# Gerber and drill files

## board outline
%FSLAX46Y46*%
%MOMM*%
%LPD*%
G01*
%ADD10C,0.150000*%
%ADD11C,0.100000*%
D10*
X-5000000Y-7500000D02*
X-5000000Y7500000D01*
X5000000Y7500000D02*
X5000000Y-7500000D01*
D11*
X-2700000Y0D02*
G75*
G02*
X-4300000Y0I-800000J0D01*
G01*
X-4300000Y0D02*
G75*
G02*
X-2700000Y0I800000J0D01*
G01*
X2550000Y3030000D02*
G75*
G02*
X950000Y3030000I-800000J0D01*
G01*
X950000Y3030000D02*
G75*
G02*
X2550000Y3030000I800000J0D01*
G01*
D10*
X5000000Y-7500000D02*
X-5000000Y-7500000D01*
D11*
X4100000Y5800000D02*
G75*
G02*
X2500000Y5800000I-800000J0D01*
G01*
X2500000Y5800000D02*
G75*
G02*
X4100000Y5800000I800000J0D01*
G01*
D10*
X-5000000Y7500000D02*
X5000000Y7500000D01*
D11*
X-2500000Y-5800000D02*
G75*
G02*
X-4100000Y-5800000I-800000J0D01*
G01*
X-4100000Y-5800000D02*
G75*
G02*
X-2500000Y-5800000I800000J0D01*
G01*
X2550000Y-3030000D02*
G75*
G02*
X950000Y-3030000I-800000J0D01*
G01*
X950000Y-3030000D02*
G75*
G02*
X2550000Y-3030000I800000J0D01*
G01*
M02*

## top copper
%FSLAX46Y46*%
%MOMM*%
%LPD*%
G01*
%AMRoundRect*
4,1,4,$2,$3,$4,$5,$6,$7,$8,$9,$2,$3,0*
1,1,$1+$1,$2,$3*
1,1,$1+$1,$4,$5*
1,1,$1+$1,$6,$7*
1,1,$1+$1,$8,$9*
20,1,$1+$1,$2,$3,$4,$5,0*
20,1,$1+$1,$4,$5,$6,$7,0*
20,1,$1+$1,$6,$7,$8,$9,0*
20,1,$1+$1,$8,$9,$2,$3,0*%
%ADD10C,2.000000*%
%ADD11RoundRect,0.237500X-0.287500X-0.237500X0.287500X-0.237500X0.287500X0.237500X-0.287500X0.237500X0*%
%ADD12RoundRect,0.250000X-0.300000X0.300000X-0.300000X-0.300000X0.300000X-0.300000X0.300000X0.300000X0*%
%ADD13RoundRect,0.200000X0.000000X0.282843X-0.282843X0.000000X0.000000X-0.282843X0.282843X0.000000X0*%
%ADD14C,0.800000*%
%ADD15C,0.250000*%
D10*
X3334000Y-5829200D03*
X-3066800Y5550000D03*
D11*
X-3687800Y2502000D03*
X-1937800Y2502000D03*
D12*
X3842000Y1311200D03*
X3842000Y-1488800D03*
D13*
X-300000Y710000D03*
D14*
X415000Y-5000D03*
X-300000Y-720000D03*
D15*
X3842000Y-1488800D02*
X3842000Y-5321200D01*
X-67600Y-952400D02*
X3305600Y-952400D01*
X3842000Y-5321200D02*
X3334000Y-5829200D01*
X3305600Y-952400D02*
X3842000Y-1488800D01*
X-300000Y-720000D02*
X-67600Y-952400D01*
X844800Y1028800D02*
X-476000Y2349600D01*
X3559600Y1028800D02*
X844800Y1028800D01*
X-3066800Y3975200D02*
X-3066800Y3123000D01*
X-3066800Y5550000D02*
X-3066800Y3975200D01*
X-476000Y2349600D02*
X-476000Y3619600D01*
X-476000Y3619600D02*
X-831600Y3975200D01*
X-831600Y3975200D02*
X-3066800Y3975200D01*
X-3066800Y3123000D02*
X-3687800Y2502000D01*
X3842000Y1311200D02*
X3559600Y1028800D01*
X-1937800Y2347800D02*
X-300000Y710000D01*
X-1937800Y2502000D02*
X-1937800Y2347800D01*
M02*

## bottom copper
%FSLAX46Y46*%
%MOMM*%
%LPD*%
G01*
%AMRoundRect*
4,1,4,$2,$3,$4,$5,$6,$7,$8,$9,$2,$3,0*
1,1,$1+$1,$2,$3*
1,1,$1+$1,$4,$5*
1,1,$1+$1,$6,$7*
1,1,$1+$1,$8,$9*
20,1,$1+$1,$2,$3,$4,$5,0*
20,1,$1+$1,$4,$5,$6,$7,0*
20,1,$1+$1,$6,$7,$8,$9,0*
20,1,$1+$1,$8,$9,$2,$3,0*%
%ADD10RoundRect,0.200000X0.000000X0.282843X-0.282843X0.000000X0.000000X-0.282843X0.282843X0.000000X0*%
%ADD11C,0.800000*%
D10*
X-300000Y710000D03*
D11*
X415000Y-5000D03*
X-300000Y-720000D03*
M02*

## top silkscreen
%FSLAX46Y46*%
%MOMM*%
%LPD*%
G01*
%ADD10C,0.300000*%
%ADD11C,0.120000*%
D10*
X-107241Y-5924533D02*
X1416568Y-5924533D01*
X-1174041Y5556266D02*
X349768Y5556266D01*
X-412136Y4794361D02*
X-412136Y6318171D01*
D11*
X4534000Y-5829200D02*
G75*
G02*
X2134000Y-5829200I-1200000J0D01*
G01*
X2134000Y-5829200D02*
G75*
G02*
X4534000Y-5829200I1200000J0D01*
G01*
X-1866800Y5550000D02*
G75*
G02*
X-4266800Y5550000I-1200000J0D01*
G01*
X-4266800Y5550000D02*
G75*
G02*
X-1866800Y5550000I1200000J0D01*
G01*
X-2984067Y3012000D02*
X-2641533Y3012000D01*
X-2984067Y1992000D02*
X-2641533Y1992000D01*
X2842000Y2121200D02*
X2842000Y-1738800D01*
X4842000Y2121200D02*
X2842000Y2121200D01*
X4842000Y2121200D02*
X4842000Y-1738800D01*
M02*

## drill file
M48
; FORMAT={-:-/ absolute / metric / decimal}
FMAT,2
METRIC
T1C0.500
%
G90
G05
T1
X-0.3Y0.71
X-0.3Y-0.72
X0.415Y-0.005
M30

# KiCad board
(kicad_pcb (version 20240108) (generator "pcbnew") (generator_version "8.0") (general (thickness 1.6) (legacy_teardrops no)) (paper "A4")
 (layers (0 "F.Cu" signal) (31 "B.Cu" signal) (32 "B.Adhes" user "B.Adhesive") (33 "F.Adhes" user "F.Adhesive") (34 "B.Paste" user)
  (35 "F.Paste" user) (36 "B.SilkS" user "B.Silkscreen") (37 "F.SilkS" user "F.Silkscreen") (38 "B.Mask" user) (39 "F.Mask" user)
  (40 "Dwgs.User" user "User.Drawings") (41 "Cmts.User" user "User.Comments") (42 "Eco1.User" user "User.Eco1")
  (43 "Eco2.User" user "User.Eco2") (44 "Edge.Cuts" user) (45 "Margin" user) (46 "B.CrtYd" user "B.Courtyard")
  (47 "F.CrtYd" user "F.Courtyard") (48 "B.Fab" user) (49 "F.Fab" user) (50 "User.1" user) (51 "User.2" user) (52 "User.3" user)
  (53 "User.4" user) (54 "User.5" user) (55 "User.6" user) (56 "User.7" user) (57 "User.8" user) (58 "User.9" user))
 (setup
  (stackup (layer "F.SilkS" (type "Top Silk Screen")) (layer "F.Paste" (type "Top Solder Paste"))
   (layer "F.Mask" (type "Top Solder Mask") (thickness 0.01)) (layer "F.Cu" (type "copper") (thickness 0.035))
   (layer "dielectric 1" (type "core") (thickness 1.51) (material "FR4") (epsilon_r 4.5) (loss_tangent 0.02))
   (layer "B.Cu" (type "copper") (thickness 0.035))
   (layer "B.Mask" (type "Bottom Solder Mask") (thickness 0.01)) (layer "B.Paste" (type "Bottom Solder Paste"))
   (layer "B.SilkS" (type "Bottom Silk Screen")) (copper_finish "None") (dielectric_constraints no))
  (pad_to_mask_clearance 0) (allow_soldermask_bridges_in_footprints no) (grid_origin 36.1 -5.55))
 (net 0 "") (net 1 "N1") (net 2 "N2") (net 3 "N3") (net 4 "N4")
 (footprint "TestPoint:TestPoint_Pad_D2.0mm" (layer "F.Cu") (at 3.334 5.8292)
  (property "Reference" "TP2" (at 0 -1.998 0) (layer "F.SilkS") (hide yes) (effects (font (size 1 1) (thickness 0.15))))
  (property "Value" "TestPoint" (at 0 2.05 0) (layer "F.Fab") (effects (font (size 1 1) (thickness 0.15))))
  (fp_circle (center 0 0) (end 0 1.2) (stroke (width 0.12) (type solid)) (fill none) (layer "F.SilkS"))
  (pad "1" smd circle (at 0 0) (size 2 2) (layers "F.Cu" "F.Mask") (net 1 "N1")))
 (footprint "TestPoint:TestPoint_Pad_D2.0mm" (layer "F.Cu") (at -3.0668 -5.55)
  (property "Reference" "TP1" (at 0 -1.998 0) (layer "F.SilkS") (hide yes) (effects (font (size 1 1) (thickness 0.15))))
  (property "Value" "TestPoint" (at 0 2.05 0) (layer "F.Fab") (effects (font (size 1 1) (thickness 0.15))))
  (fp_circle (center 0 0) (end 0 1.2) (stroke (width 0.12) (type solid)) (fill none) (layer "F.SilkS"))
  (pad "1" smd circle (at 0 0) (size 2 2) (layers "F.Cu" "F.Mask") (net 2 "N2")))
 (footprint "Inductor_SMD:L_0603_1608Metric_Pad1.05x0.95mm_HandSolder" (layer "F.Cu") (at -2.8128 -2.502)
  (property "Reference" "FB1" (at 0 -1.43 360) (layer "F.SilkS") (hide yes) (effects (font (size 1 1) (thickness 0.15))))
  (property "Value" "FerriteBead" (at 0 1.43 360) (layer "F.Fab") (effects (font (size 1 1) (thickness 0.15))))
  (fp_line (start -0.171267 -0.51) (end 0.171267 -0.51) (stroke (width 0.12) (type solid)) (layer "F.SilkS"))
  (fp_line (start -0.171267 0.51) (end 0.171267 0.51) (stroke (width 0.12) (type solid)) (layer "F.SilkS"))
  (pad "1" smd roundrect (at -0.875 0) (size 1.05 0.95) (layers "F.Cu" "F.Paste" "F.Mask") (roundrect_rratio 0.25) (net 2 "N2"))
  (pad "2" smd roundrect (at 0.875 0) (size 1.05 0.95) (layers "F.Cu" "F.Paste" "F.Mask") (roundrect_rratio 0.25) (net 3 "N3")))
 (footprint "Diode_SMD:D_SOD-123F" (layer "F.Cu") (at 3.842 0.0888 -90)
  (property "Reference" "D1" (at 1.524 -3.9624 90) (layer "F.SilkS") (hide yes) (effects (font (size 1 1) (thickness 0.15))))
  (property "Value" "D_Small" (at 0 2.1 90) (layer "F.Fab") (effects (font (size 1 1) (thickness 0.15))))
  (fp_line (start -2.21 1) (end 1.65 1) (stroke (width 0.12) (type solid)) (layer "F.SilkS"))
  (fp_line (start -2.21 -1) (end -2.21 1) (stroke (width 0.12) (type solid)) (layer "F.SilkS"))
  (fp_line (start -2.21 -1) (end 1.65 -1) (stroke (width 0.12) (type solid)) (layer "F.SilkS"))
  (pad "1" smd roundrect (at -1.4 0 270) (size 1.1 1.1) (layers "F.Cu" "F.Paste" "F.Mask") (roundrect_rratio 0.2272727273) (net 2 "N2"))
  (pad "2" smd roundrect (at 1.4 0 270) (size 1.1 1.1) (layers "F.Cu" "F.Paste" "F.Mask") (roundrect_rratio 0.2272727273) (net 1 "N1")))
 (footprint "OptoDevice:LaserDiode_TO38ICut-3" (layer "B.Cu") (at 0 0 -90)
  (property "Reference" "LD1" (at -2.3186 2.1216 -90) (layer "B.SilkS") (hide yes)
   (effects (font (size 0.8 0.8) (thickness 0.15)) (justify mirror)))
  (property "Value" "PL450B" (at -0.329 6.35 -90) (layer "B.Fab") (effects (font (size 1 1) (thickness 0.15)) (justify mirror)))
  (pad "1" thru_hole roundrect (at -0.71 0.3 225) (size 0.8 0.8) (drill 0.5) (layers "*.Cu" "*.Mask") (remove_unused_layers no)
   (roundrect_rratio 0.25) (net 3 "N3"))
  (pad "2" thru_hole circle (at 0.005 -0.415 270) (size 0.8 0.8) (drill 0.5) (layers "*.Cu" "*.Mask") (remove_unused_layers no) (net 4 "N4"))
  (pad "3" thru_hole circle (at 0.72 0.3 270) (size 0.8 0.8) (drill 0.5) (layers "*.Cu" "*.Mask") (remove_unused_layers no) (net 1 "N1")))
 (gr_line (start -5 7.5) (end -5 -7.5) (stroke (width 0.15) (type default)) (layer "Edge.Cuts"))
 (gr_line (start 5 -7.5) (end 5 7.5) (stroke (width 0.15) (type default)) (layer "Edge.Cuts"))
 (gr_circle (center -3.5 0) (end -2.7 0) (stroke (width 0.1) (type default)) (fill none) (layer "Edge.Cuts"))
 (gr_circle (center 1.75 -3.03) (end 2.55 -3.03) (stroke (width 0.1) (type default)) (fill none) (layer "Edge.Cuts"))
 (gr_line (start 5 7.5) (end -5 7.5) (stroke (width 0.15) (type default)) (layer "Edge.Cuts"))
 (gr_circle (center 3.3 -5.8) (end 4.1 -5.8) (stroke (width 0.1) (type default)) (fill none) (layer "Edge.Cuts"))
 (gr_line (start -5 -7.5) (end 5 -7.5) (stroke (width 0.15) (type default)) (layer "Edge.Cuts"))
 (gr_circle (center -3.3 5.8) (end -2.5 5.8) (stroke (width 0.1) (type default)) (fill none) (layer "Edge.Cuts"))
 (gr_circle (center 1.75 3.03) (end 2.55 3.03) (stroke (width 0.1) (type default)) (fill none) (layer "Edge.Cuts"))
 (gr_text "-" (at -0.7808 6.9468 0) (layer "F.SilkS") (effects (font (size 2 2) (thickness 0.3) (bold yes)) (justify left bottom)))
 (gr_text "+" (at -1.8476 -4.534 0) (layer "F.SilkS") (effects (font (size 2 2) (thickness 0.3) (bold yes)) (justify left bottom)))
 (segment (start 3.842 1.4888) (end 3.842 5.3212) (width 0.25) (layer "F.Cu") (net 1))
 (segment (start -0.0676 0.9524) (end 3.3056 0.9524) (width 0.25) (layer "F.Cu") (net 1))
 (segment (start 3.842 5.3212) (end 3.334 5.8292) (width 0.25) (layer "F.Cu") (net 1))
 (segment (start 3.3056 0.9524) (end 3.842 1.4888) (width 0.25) (layer "F.Cu") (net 1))
 (segment (start -0.3 0.72) (end -0.0676 0.9524) (width 0.25) (layer "F.Cu") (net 1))
 (segment (start 0.8448 -1.0288) (end -0.476 -2.3496) (width 0.25) (layer "F.Cu") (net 2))
 (segment (start 3.5596 -1.0288) (end 0.8448 -1.0288) (width 0.25) (layer "F.Cu") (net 2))
 (segment (start -3.0668 -3.9752) (end -3.0668 -3.123) (width 0.25) (layer "F.Cu") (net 2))
 (segment (start -3.0668 -5.55) (end -3.0668 -3.9752) (width 0.25) (layer "F.Cu") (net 2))
 (segment (start -0.476 -2.3496) (end -0.476 -3.6196) (width 0.25) (layer "F.Cu") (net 2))
 (segment (start -0.476 -3.6196) (end -0.8316 -3.9752) (width 0.25) (layer "F.Cu") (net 2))
 (segment (start -0.8316 -3.9752) (end -3.0668 -3.9752) (width 0.25) (layer "F.Cu") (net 2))
 (segment (start -3.0668 -3.123) (end -3.6878 -2.502) (width 0.25) (layer "F.Cu") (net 2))
 (segment (start 3.842 -1.3112) (end 3.5596 -1.0288) (width 0.25) (layer "F.Cu") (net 2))
 (segment (start -1.9378 -2.3478) (end -0.3 -0.71) (width 0.25) (layer "F.Cu") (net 3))
 (segment (start -1.9378 -2.502) (end -1.9378 -2.3478) (width 0.25) (layer "F.Cu") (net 3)))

